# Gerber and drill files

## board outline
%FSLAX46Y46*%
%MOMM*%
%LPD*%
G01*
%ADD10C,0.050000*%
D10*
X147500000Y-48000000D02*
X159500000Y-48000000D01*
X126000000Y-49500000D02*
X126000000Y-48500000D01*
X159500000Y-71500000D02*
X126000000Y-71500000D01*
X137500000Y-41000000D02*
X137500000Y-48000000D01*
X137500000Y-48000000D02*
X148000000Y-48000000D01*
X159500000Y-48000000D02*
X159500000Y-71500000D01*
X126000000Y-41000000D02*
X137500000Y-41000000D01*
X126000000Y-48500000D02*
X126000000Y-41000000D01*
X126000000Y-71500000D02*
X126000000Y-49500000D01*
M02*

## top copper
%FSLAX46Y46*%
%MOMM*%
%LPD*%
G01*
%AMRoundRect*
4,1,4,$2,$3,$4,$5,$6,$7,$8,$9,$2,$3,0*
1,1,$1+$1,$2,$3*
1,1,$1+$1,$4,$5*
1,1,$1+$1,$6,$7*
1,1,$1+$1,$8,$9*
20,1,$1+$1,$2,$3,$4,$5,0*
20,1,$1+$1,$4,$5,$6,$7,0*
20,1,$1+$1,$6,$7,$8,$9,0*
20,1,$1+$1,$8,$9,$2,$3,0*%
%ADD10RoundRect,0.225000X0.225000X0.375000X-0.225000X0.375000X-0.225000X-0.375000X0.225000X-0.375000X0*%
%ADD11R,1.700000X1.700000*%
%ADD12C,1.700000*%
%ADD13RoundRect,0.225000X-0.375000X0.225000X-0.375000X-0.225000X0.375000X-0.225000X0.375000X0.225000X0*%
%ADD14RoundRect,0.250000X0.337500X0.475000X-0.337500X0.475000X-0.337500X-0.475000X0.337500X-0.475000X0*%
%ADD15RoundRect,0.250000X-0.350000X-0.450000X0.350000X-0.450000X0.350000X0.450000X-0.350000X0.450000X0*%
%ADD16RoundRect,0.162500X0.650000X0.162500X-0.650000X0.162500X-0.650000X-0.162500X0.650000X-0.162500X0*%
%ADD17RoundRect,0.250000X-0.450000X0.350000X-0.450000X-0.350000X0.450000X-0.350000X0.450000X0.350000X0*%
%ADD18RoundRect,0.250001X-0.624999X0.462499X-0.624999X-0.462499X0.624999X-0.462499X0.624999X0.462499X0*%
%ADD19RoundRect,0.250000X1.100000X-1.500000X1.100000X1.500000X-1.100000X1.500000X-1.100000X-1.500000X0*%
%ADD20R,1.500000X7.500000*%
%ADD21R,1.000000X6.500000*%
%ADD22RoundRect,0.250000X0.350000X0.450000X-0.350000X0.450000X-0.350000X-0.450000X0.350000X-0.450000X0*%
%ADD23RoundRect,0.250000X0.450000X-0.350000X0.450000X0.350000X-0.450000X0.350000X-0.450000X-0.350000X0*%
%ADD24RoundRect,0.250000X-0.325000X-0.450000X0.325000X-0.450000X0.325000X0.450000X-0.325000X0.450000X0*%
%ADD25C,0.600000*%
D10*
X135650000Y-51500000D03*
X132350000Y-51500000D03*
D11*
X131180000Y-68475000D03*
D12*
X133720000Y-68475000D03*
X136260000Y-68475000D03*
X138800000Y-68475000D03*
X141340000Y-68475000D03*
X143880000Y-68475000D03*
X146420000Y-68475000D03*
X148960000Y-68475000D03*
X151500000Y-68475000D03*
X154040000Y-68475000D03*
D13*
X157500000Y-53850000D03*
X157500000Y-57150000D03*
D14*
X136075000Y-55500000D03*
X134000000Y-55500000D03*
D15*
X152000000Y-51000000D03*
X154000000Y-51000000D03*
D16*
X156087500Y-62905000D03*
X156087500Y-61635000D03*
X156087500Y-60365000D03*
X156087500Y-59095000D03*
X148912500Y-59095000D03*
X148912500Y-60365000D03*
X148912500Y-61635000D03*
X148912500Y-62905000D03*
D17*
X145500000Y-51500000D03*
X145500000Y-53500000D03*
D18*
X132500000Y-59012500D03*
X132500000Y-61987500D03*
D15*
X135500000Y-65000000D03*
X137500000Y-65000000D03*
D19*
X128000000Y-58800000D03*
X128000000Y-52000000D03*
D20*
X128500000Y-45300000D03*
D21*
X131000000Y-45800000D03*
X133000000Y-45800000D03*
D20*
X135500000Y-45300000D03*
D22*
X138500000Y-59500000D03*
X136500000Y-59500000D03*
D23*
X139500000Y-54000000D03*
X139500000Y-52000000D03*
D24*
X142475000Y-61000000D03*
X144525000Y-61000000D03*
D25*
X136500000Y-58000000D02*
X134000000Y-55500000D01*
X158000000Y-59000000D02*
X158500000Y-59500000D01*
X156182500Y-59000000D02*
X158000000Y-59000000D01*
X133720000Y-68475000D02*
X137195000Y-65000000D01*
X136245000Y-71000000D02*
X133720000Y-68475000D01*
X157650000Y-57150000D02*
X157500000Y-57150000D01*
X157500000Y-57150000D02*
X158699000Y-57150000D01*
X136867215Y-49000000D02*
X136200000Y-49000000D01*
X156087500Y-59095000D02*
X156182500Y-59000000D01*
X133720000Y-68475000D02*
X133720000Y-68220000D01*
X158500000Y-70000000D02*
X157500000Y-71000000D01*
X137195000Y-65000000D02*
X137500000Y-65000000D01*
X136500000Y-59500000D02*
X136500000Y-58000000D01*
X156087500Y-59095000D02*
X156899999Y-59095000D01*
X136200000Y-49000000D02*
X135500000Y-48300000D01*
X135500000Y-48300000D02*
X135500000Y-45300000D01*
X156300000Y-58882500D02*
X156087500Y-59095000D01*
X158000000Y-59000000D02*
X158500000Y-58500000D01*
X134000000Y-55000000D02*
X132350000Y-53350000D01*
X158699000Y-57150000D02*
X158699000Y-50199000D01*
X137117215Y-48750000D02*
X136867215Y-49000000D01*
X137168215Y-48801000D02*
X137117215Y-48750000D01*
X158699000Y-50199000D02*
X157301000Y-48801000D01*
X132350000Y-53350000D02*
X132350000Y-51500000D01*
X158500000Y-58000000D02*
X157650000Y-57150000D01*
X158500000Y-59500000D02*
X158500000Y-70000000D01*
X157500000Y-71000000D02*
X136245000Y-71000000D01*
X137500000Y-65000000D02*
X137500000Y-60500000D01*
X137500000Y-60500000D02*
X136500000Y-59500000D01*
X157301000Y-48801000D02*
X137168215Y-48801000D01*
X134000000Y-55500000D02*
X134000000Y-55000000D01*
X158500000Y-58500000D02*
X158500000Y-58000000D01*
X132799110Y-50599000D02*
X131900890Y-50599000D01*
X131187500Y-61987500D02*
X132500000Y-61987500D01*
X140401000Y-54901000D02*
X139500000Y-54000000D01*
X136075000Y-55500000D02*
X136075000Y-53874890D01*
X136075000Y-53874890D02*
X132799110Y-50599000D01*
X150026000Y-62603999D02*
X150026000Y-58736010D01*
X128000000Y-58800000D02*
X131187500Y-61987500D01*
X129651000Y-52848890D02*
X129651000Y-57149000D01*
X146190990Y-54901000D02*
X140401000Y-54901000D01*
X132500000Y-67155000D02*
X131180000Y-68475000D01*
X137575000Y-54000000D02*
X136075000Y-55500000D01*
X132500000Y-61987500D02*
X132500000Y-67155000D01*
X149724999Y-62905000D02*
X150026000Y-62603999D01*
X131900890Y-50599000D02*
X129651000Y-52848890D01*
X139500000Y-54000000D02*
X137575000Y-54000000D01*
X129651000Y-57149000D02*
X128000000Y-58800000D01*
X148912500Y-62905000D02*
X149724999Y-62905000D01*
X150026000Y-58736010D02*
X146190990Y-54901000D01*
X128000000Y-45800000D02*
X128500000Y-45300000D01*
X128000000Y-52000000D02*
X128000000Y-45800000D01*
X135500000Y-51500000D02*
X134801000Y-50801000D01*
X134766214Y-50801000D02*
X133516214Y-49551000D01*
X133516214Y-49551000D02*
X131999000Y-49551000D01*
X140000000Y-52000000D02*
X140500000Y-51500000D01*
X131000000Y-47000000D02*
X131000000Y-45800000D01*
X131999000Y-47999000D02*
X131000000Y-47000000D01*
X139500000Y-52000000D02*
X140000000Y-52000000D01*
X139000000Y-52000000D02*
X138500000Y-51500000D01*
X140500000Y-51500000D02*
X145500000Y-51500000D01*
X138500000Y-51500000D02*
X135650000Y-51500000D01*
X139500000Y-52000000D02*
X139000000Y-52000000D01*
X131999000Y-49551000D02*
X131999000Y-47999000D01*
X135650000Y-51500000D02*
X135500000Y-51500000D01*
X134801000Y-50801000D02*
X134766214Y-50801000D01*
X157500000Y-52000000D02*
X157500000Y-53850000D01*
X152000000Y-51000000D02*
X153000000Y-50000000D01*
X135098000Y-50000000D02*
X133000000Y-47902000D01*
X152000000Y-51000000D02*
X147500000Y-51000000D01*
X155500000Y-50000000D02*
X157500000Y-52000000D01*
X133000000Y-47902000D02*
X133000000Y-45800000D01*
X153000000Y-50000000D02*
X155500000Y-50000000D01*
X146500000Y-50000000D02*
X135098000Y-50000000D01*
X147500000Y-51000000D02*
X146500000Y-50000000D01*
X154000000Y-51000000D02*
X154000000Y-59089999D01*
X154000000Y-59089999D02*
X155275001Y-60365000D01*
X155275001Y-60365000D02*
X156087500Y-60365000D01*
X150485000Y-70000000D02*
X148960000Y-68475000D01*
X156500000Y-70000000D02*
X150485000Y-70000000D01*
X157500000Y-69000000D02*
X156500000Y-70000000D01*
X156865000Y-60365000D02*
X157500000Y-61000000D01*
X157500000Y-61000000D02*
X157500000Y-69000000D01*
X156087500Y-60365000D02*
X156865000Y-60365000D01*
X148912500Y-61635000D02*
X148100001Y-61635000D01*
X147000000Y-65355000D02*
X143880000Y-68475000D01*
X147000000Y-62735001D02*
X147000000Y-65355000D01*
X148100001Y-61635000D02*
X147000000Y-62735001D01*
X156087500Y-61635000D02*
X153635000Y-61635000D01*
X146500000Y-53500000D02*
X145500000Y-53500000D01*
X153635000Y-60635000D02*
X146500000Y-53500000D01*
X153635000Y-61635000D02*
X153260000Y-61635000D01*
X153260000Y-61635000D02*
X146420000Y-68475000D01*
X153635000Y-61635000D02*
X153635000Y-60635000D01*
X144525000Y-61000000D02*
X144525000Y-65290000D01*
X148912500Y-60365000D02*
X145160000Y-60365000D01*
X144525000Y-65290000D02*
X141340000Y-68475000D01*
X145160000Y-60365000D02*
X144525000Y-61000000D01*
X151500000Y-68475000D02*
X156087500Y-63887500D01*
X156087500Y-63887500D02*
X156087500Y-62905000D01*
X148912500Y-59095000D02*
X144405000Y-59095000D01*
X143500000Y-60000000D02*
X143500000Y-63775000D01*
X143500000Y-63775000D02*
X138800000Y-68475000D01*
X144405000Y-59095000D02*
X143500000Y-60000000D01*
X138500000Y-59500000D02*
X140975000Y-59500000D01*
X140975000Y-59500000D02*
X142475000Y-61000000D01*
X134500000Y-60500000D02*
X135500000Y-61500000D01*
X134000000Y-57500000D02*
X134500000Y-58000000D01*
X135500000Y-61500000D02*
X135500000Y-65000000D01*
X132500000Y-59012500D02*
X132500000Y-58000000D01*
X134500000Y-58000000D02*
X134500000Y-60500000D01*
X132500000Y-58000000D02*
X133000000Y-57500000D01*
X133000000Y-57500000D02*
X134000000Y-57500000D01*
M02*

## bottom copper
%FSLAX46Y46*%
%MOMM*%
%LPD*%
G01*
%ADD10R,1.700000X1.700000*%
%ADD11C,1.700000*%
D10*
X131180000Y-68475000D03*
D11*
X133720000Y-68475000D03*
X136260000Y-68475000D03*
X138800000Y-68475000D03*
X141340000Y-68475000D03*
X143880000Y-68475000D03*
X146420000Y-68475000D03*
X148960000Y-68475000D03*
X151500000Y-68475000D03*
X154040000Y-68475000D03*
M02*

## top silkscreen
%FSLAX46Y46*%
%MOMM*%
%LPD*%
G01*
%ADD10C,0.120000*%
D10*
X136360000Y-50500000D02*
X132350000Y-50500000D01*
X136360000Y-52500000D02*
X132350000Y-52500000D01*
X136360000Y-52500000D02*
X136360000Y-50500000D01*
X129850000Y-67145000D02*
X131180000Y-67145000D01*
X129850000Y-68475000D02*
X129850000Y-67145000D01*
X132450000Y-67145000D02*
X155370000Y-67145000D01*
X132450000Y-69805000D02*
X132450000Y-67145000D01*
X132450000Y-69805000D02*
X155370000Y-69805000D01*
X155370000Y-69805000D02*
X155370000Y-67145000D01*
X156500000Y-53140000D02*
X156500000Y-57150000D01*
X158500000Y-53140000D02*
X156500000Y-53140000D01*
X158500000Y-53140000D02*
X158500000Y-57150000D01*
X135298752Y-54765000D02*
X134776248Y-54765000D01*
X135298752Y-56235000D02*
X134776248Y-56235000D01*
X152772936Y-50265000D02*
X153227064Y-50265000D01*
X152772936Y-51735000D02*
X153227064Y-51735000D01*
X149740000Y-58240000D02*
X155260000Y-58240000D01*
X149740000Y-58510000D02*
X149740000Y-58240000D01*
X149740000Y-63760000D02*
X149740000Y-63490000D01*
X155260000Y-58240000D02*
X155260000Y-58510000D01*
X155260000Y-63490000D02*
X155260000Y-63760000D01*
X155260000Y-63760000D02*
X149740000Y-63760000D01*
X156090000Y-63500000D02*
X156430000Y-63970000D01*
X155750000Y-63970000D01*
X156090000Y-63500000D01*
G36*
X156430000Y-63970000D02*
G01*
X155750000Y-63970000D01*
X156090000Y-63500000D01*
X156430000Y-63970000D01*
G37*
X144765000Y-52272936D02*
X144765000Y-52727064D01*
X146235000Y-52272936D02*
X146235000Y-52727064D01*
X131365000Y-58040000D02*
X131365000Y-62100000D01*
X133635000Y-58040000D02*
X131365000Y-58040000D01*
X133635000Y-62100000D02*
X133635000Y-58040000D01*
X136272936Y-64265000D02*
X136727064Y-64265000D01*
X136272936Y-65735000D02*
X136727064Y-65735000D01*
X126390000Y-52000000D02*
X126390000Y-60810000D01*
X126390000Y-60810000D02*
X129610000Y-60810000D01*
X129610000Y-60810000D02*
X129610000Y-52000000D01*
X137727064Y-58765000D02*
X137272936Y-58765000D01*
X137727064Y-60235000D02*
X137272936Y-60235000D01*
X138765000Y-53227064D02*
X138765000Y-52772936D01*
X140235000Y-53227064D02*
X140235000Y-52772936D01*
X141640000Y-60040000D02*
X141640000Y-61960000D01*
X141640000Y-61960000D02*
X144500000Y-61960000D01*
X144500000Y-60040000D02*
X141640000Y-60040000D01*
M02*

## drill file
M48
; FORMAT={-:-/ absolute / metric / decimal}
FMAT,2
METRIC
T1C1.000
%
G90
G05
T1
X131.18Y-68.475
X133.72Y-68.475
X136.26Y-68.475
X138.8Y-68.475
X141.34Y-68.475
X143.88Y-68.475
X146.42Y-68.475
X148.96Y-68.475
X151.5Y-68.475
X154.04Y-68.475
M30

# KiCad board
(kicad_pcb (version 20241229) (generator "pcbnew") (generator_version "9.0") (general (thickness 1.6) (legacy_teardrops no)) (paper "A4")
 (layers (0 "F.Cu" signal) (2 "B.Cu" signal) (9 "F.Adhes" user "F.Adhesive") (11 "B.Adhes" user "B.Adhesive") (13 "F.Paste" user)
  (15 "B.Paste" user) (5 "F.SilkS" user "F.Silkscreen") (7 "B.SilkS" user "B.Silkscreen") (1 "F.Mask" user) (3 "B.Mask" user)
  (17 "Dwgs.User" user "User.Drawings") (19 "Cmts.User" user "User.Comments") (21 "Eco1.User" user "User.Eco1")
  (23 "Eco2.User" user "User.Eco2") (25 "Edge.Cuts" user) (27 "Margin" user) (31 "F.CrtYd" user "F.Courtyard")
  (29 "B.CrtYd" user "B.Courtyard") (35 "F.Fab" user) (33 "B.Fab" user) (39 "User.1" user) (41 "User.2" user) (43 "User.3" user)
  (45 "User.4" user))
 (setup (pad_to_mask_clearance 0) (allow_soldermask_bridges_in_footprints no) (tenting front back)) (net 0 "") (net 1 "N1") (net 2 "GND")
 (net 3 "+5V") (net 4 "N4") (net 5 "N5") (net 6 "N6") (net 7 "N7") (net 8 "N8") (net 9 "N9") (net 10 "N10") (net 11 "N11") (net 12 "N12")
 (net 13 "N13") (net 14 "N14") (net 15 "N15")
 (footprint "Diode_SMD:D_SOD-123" (layer "F.Cu") (at 134 51.5 180)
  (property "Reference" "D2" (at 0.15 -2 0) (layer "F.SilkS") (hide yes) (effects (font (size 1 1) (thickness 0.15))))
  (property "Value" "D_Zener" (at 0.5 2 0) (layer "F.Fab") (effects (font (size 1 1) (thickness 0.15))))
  (fp_line (start -2.36 1) (end 1.65 1) (stroke (width 0.12) (type solid)) (layer "F.SilkS"))
  (fp_line (start -2.36 -1) (end 1.65 -1) (stroke (width 0.12) (type solid)) (layer "F.SilkS"))
  (fp_line (start -2.36 -1) (end -2.36 1) (stroke (width 0.12) (type solid)) (layer "F.SilkS"))
  (pad "1" smd roundrect (at -1.65 0 180) (size 0.9 1.2) (layers "F.Cu" "F.Mask" "F.Paste") (roundrect_rratio 0.25) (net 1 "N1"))
  (pad "2" smd roundrect (at 1.65 0 180) (size 0.9 1.2) (layers "F.Cu" "F.Mask" "F.Paste") (roundrect_rratio 0.25) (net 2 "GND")))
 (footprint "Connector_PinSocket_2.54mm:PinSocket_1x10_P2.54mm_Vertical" (layer "F.Cu") (at 131.18 68.475 90)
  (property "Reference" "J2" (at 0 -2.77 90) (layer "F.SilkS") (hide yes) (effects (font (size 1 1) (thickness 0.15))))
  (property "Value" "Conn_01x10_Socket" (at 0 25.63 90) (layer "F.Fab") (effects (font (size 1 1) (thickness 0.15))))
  (fp_line (start 1.33 -1.33) (end 1.33 0) (stroke (width 0.12) (type solid)) (layer "F.SilkS"))
  (fp_line (start 0 -1.33) (end 1.33 -1.33) (stroke (width 0.12) (type solid)) (layer "F.SilkS"))
  (fp_line (start 1.33 1.27) (end 1.33 24.19) (stroke (width 0.12) (type solid)) (layer "F.SilkS"))
  (fp_line (start -1.33 1.27) (end 1.33 1.27) (stroke (width 0.12) (type solid)) (layer "F.SilkS"))
  (fp_line (start -1.33 1.27) (end -1.33 24.19) (stroke (width 0.12) (type solid)) (layer "F.SilkS"))
  (fp_line (start -1.33 24.19) (end 1.33 24.19) (stroke (width 0.12) (type solid)) (layer "F.SilkS"))
  (pad "1" thru_hole rect (at 0 0 90) (size 1.7 1.7) (drill 1) (layers "*.Cu" "*.Mask") (remove_unused_layers no) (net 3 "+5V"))
  (pad "2" thru_hole circle (at 0 2.54 90) (size 1.7 1.7) (drill 1) (layers "*.Cu" "*.Mask") (remove_unused_layers no) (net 2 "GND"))
  (pad "3" thru_hole circle (at 0 5.08 90) (size 1.7 1.7) (drill 1) (layers "*.Cu" "*.Mask") (remove_unused_layers no) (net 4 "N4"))
  (pad "4" thru_hole circle (at 0 7.62 90) (size 1.7 1.7) (drill 1) (layers "*.Cu" "*.Mask") (remove_unused_layers no) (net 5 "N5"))
  (pad "5" thru_hole circle (at 0 10.16 90) (size 1.7 1.7) (drill 1) (layers "*.Cu" "*.Mask") (remove_unused_layers no) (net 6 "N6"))
  (pad "6" thru_hole circle (at 0 12.7 90) (size 1.7 1.7) (drill 1) (layers "*.Cu" "*.Mask") (remove_unused_layers no) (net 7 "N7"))
  (pad "7" thru_hole circle (at 0 15.24 90) (size 1.7 1.7) (drill 1) (layers "*.Cu" "*.Mask") (remove_unused_layers no) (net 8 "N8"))
  (pad "8" thru_hole circle (at 0 17.78 90) (size 1.7 1.7) (drill 1) (layers "*.Cu" "*.Mask") (remove_unused_layers no) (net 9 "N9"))
  (pad "9" thru_hole circle (at 0 20.32 90) (size 1.7 1.7) (drill 1) (layers "*.Cu" "*.Mask") (remove_unused_layers no) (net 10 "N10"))
  (pad "10" thru_hole circle (at 0 22.86 90) (size 1.7 1.7) (drill 1) (layers "*.Cu" "*.Mask") (remove_unused_layers no) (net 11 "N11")))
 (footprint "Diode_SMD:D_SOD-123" (layer "F.Cu") (at 157.5 55.5 -90)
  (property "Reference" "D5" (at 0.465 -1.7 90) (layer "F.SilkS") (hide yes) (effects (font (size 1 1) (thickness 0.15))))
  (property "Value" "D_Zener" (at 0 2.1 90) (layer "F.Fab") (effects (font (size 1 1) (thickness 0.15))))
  (fp_line (start -2.36 1) (end 1.65 1) (stroke (width 0.12) (type solid)) (layer "F.SilkS"))
  (fp_line (start -2.36 -1) (end -2.36 1) (stroke (width 0.12) (type solid)) (layer "F.SilkS"))
  (fp_line (start -2.36 -1) (end 1.65 -1) (stroke (width 0.12) (type solid)) (layer "F.SilkS"))
  (pad "1" smd roundrect (at -1.65 0 270) (size 0.9 1.2) (layers "F.Cu" "F.Mask" "F.Paste") (roundrect_rratio 0.25) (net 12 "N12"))
  (pad "2" smd roundrect (at 1.65 0 270) (size 0.9 1.2) (layers "F.Cu" "F.Mask" "F.Paste") (roundrect_rratio 0.25) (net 2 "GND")))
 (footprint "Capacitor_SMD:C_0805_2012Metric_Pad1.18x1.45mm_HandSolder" (layer "F.Cu") (at 135.0375 55.5 180)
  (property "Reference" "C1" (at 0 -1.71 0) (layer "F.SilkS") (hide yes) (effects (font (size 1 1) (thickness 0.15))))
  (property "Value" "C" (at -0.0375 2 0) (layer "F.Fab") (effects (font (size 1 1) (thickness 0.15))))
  (fp_line (start -0.261252 0.735) (end 0.261252 0.735) (stroke (width 0.12) (type solid)) (layer "F.SilkS"))
  (fp_line (start -0.261252 -0.735) (end 0.261252 -0.735) (stroke (width 0.12) (type solid)) (layer "F.SilkS"))
  (pad "1" smd roundrect (at -1.0375 0 180) (size 1.175 1.45) (layers "F.Cu" "F.Mask" "F.Paste") (roundrect_rratio 0.212766) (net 3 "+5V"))
  (pad "2" smd roundrect (at 1.0375 0 180) (size 1.175 1.45) (layers "F.Cu" "F.Mask" "F.Paste") (roundrect_rratio 0.212766) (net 2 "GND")))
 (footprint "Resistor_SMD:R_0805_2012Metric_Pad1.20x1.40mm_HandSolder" (layer "F.Cu") (at 153 51)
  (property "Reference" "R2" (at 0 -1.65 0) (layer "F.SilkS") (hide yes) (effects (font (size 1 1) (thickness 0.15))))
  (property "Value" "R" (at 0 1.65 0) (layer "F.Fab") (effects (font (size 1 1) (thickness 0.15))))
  (fp_line (start -0.227064 -0.735) (end 0.227064 -0.735) (stroke (width 0.12) (type solid)) (layer "F.SilkS"))
  (fp_line (start -0.227064 0.735) (end 0.227064 0.735) (stroke (width 0.12) (type solid)) (layer "F.SilkS"))
  (pad "1" smd roundrect (at -1 0) (size 1.2 1.4) (layers "F.Cu" "F.Mask" "F.Paste") (roundrect_rratio 0.208333) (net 12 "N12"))
  (pad "2" smd roundrect (at 1 0) (size 1.2 1.4) (layers "F.Cu" "F.Mask" "F.Paste") (roundrect_rratio 0.208333) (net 9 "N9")))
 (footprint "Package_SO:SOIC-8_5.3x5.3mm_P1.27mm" (layer "F.Cu") (at 152.5 61 180)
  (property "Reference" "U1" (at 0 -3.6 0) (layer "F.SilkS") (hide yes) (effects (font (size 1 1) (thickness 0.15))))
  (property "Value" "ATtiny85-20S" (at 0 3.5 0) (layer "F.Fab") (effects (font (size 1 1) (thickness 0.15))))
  (fp_line (start 2.76 2.76) (end -2.76 2.76) (stroke (width 0.12) (type solid)) (layer "F.SilkS"))
  (fp_line (start 2.76 2.49) (end 2.76 2.76) (stroke (width 0.12) (type solid)) (layer "F.SilkS"))
  (fp_line (start 2.76 -2.76) (end 2.76 -2.49) (stroke (width 0.12) (type solid)) (layer "F.SilkS"))
  (fp_line (start -2.76 2.76) (end -2.76 2.49) (stroke (width 0.12) (type solid)) (layer "F.SilkS"))
  (fp_line (start -2.76 -2.49) (end -2.76 -2.76) (stroke (width 0.12) (type solid)) (layer "F.SilkS"))
  (fp_line (start -2.76 -2.76) (end 2.76 -2.76) (stroke (width 0.12) (type solid)) (layer "F.SilkS"))
  (fp_poly (pts (xy -3.59 -2.5) (xy -3.93 -2.97) (xy -3.25 -2.97)) (stroke (width 0.12) (type solid)) (fill yes) (layer "F.SilkS"))
  (pad "1" smd roundrect (at -3.5875 -1.905 180) (size 1.625 0.65) (layers "F.Cu" "F.Mask" "F.Paste") (roundrect_rratio 0.25) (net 10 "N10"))
  (pad "2" smd roundrect (at -3.5875 -0.635 180) (size 1.625 0.65) (layers "F.Cu" "F.Mask" "F.Paste") (roundrect_rratio 0.25) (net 8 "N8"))
  (pad "3" smd roundrect (at -3.5875 0.635 180) (size 1.625 0.65) (layers "F.Cu" "F.Mask" "F.Paste") (roundrect_rratio 0.25) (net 9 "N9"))
  (pad "4" smd roundrect (at -3.5875 1.905 180) (size 1.625 0.65) (layers "F.Cu" "F.Mask" "F.Paste") (roundrect_rratio 0.25) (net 2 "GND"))
  (pad "5" smd roundrect (at 3.5875 1.905 180) (size 1.625 0.65) (layers "F.Cu" "F.Mask" "F.Paste") (roundrect_rratio 0.25) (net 5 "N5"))
  (pad "6" smd roundrect (at 3.5875 0.635 180) (size 1.625 0.65) (layers "F.Cu" "F.Mask" "F.Paste") (roundrect_rratio 0.25) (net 6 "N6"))
  (pad "7" smd roundrect (at 3.5875 -0.635 180) (size 1.625 0.65) (layers "F.Cu" "F.Mask" "F.Paste") (roundrect_rratio 0.25) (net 7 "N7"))
  (pad "8" smd roundrect (at 3.5875 -1.905 180) (size 1.625 0.65) (layers "F.Cu" "F.Mask" "F.Paste") (roundrect_rratio 0.25) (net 3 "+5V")))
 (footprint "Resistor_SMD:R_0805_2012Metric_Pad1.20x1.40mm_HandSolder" (layer "F.Cu") (at 145.5 52.5 -90)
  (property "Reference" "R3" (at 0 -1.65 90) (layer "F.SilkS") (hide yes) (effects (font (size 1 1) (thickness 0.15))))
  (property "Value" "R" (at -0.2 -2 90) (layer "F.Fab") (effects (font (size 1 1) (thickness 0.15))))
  (fp_line (start -0.227064 0.735) (end 0.227064 0.735) (stroke (width 0.12) (type solid)) (layer "F.SilkS"))
  (fp_line (start -0.227064 -0.735) (end 0.227064 -0.735) (stroke (width 0.12) (type solid)) (layer "F.SilkS"))
  (pad "1" smd roundrect (at -1 0 270) (size 1.2 1.4) (layers "F.Cu" "F.Mask" "F.Paste") (roundrect_rratio 0.208333) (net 1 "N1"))
  (pad "2" smd roundrect (at 1 0 270) (size 1.2 1.4) (layers "F.Cu" "F.Mask" "F.Paste") (roundrect_rratio 0.208333) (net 8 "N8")))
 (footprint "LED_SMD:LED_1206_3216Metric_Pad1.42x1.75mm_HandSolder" (layer "F.Cu") (at 132.5 60.5 -90)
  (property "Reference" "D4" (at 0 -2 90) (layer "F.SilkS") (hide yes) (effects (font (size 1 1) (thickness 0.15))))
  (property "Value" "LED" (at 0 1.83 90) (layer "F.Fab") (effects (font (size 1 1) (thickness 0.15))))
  (fp_line (start -2.46 1.135) (end 1.6 1.135) (stroke (width 0.12) (type solid)) (layer "F.SilkS"))
  (fp_line (start -2.46 -1.135) (end -2.46 1.135) (stroke (width 0.12) (type solid)) (layer "F.SilkS"))
  (fp_line (start 1.6 -1.135) (end -2.46 -1.135) (stroke (width 0.12) (type solid)) (layer "F.SilkS"))
  (pad "1" smd roundrect (at -1.4875 0 270) (size 1.425 1.75) (layers "F.Cu" "F.Mask" "F.Paste") (roundrect_rratio 0.175439) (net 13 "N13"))
  (pad "2" smd roundrect (at 1.4875 0 270) (size 1.425 1.75) (layers "F.Cu" "F.Mask" "F.Paste") (roundrect_rratio 0.175439) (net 3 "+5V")))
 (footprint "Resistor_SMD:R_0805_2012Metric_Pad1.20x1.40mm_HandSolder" (layer "F.Cu") (at 136.5 65)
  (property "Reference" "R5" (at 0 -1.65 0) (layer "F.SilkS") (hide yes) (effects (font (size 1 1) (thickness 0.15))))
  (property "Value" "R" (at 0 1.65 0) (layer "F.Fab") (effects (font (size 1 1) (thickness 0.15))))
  (fp_line (start -0.227064 -0.735) (end 0.227064 -0.735) (stroke (width 0.12) (type solid)) (layer "F.SilkS"))
  (fp_line (start -0.227064 0.735) (end 0.227064 0.735) (stroke (width 0.12) (type solid)) (layer "F.SilkS"))
  (pad "1" smd roundrect (at -1 0) (size 1.2 1.4) (layers "F.Cu" "F.Mask" "F.Paste") (roundrect_rratio 0.208333) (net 13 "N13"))
  (pad "2" smd roundrect (at 1 0) (size 1.2 1.4) (layers "F.Cu" "F.Mask" "F.Paste") (roundrect_rratio 0.208333) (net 2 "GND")))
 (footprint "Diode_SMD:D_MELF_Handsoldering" (layer "F.Cu") (at 128 55.4 90)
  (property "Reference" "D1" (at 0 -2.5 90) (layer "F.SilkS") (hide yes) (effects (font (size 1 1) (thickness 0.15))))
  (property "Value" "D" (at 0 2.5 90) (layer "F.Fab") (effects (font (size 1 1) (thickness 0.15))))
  (fp_line (start 3.4 -1.61) (end -5.41 -1.61) (stroke (width 0.12) (type solid)) (layer "F.SilkS"))
  (fp_line (start -5.41 -1.61) (end -5.41 1.61) (stroke (width 0.12) (type solid)) (layer "F.SilkS"))
  (fp_line (start -5.41 1.61) (end 3.4 1.61) (stroke (width 0.12) (type solid)) (layer "F.SilkS"))
  (pad "1" smd roundrect (at -3.4 0 90) (size 3.5 2.7) (layers "F.Cu" "F.Mask" "F.Paste") (roundrect_rratio 0.0925925926) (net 3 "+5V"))
  (pad "2" smd roundrect (at 3.4 0 90) (size 3.5 2.7) (layers "F.Cu" "F.Mask" "F.Paste") (roundrect_rratio 0.0925925926) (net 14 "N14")))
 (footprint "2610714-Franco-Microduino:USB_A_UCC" (layer "F.Cu") (at 132 45.5 -90)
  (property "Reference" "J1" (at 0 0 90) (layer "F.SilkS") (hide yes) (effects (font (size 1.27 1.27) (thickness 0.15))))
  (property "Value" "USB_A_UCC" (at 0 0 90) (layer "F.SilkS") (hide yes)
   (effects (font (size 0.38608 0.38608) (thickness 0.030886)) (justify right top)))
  (pad "1" smd rect (at -0.2 3.5 270) (size 7.5 1.5) (layers "F.Cu" "F.Mask" "F.Paste") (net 14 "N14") (solder_mask_margin 0.1016))
  (pad "2" smd rect (at 0.3 1 270) (size 6.5 1) (layers "F.Cu" "F.Mask" "F.Paste") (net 1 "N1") (solder_mask_margin 0.1016))
  (pad "3" smd rect (at 0.3 -1 270) (size 6.5 1) (layers "F.Cu" "F.Mask" "F.Paste") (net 12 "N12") (solder_mask_margin 0.1016))
  (pad "4" smd rect (at -0.2 -3.5 270) (size 7.5 1.5) (layers "F.Cu" "F.Mask" "F.Paste") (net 2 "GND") (solder_mask_margin 0.1016)))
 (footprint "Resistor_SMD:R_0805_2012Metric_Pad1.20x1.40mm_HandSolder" (layer "F.Cu") (at 137.5 59.5 180)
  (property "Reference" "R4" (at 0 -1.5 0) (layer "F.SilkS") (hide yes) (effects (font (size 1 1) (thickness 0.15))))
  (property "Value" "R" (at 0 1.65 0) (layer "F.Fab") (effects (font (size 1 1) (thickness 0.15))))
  (fp_line (start -0.227064 0.735) (end 0.227064 0.735) (stroke (width 0.12) (type solid)) (layer "F.SilkS"))
  (fp_line (start -0.227064 -0.735) (end 0.227064 -0.735) (stroke (width 0.12) (type solid)) (layer "F.SilkS"))
  (pad "1" smd roundrect (at -1 0 180) (size 1.2 1.4) (layers "F.Cu" "F.Mask" "F.Paste") (roundrect_rratio 0.208333) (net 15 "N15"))
  (pad "2" smd roundrect (at 1 0 180) (size 1.2 1.4) (layers "F.Cu" "F.Mask" "F.Paste") (roundrect_rratio 0.208333) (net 2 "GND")))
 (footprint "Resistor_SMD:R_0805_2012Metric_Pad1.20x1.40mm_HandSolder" (layer "F.Cu") (at 139.5 53 90)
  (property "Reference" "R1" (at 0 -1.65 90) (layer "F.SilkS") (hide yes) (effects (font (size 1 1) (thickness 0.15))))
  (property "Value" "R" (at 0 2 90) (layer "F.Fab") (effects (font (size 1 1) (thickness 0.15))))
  (fp_line (start -0.227064 -0.735) (end 0.227064 -0.735) (stroke (width 0.12) (type solid)) (layer "F.SilkS"))
  (fp_line (start -0.227064 0.735) (end 0.227064 0.735) (stroke (width 0.12) (type solid)) (layer "F.SilkS"))
  (pad "1" smd roundrect (at -1 0 90) (size 1.2 1.4) (layers "F.Cu" "F.Mask" "F.Paste") (roundrect_rratio 0.208333) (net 3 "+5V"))
  (pad "2" smd roundrect (at 1 0 90) (size 1.2 1.4) (layers "F.Cu" "F.Mask" "F.Paste") (roundrect_rratio 0.208333) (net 1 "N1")))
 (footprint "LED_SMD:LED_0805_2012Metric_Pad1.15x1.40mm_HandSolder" (layer "F.Cu") (at 143.5 61)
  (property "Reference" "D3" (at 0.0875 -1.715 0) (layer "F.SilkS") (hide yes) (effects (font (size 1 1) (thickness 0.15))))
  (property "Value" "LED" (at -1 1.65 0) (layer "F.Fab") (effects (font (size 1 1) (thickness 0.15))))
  (fp_line (start -1.86 -0.96) (end -1.86 0.96) (stroke (width 0.12) (type solid)) (layer "F.SilkS"))
  (fp_line (start -1.86 0.96) (end 1 0.96) (stroke (width 0.12) (type solid)) (layer "F.SilkS"))
  (fp_line (start 1 -0.96) (end -1.86 -0.96) (stroke (width 0.12) (type solid)) (layer "F.SilkS"))
  (pad "1" smd roundrect (at -1.025 0) (size 1.15 1.4) (layers "F.Cu" "F.Mask" "F.Paste") (roundrect_rratio 0.217391) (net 15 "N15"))
  (pad "2" smd roundrect (at 1.025 0) (size 1.15 1.4) (layers "F.Cu" "F.Mask" "F.Paste") (roundrect_rratio 0.217391) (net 6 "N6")))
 (gr_line (start 147.5 48) (end 159.5 48) (stroke (width 0.05) (type default)) (layer "Edge.Cuts"))
 (gr_line (start 126 49.5) (end 126 48.5) (stroke (width 0.05) (type default)) (layer "Edge.Cuts"))
 (gr_line (start 159.5 71.5) (end 126 71.5) (stroke (width 0.05) (type default)) (layer "Edge.Cuts"))
 (gr_line (start 137.5 41) (end 137.5 48) (stroke (width 0.05) (type default)) (layer "Edge.Cuts"))
 (gr_line (start 137.5 48) (end 148 48) (stroke (width 0.05) (type default)) (layer "Edge.Cuts"))
 (gr_line (start 159.5 48) (end 159.5 71.5) (stroke (width 0.05) (type default)) (layer "Edge.Cuts"))
 (gr_line (start 126 41) (end 137.5 41) (stroke (width 0.05) (type default)) (layer "Edge.Cuts"))
 (gr_line (start 126 48.5) (end 126 41) (stroke (width 0.05) (type default)) (layer "Edge.Cuts"))
 (gr_line (start 126 71.5) (end 126 49.5) (stroke (width 0.05) (type default)) (layer "Edge.Cuts"))
 (segment (start 136.5 58) (end 134 55.5) (width 0.6) (layer "F.Cu") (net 2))
 (segment (start 158 59) (end 158.5 59.5) (width 0.6) (layer "F.Cu") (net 2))
 (segment (start 156.1825 59) (end 158 59) (width 0.6) (layer "F.Cu") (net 2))
 (segment (start 133.72 68.475) (end 137.195 65) (width 0.6) (layer "F.Cu") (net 2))
 (segment (start 136.245 71) (end 133.72 68.475) (width 0.6) (layer "F.Cu") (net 2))
 (segment (start 157.65 57.15) (end 157.5 57.15) (width 0.6) (layer "F.Cu") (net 2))
 (segment (start 157.5 57.15) (end 158.699 57.15) (width 0.6) (layer "F.Cu") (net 2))
 (segment (start 136.867215 49) (end 136.2 49) (width 0.6) (layer "F.Cu") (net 2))
 (segment (start 156.0875 59.095) (end 156.1825 59) (width 0.6) (layer "F.Cu") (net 2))
 (segment (start 133.72 68.475) (end 133.72 68.22) (width 0.6) (layer "F.Cu") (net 2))
 (segment (start 158.5 70) (end 157.5 71) (width 0.6) (layer "F.Cu") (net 2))
 (segment (start 137.195 65) (end 137.5 65) (width 0.6) (layer "F.Cu") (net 2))
 (segment (start 136.5 59.5) (end 136.5 58) (width 0.6) (layer "F.Cu") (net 2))
 (segment (start 156.0875 59.095) (end 156.899999 59.095) (width 0.6) (layer "F.Cu") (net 2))
 (segment (start 136.2 49) (end 135.5 48.3) (width 0.6) (layer "F.Cu") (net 2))
 (segment (start 135.5 48.3) (end 135.5 45.3) (width 0.6) (layer "F.Cu") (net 2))
 (segment (start 156.3 58.8825) (end 156.0875 59.095) (width 0.6) (layer "F.Cu") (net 2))
 (segment (start 158 59) (end 158.5 58.5) (width 0.6) (layer "F.Cu") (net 2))
 (segment (start 134 55) (end 132.35 53.35) (width 0.6) (layer "F.Cu") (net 2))
 (segment (start 158.699 57.15) (end 158.699 50.199) (width 0.6) (layer "F.Cu") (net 2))
 (segment (start 137.117215 48.75) (end 136.867215 49) (width 0.6) (layer "F.Cu") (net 2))
 (segment (start 137.168215 48.801) (end 137.117215 48.75) (width 0.6) (layer "F.Cu") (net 2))
 (segment (start 158.699 50.199) (end 157.301 48.801) (width 0.6) (layer "F.Cu") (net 2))
 (segment (start 132.35 53.35) (end 132.35 51.5) (width 0.6) (layer "F.Cu") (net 2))
 (segment (start 158.5 58) (end 157.65 57.15) (width 0.6) (layer "F.Cu") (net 2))
 (segment (start 158.5 59.5) (end 158.5 70) (width 0.6) (layer "F.Cu") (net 2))
 (segment (start 157.5 71) (end 136.245 71) (width 0.6) (layer "F.Cu") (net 2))
 (segment (start 137.5 65) (end 137.5 60.5) (width 0.6) (layer "F.Cu") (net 2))
 (segment (start 137.5 60.5) (end 136.5 59.5) (width 0.6) (layer "F.Cu") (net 2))
 (segment (start 157.301 48.801) (end 137.168215 48.801) (width 0.6) (layer "F.Cu") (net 2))
 (segment (start 134 55.5) (end 134 55) (width 0.6) (layer "F.Cu") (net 2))
 (segment (start 158.5 58.5) (end 158.5 58) (width 0.6) (layer "F.Cu") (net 2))
 (segment (start 132.79911 50.599) (end 131.90089 50.599) (width 0.6) (layer "F.Cu") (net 3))
 (segment (start 131.1875 61.9875) (end 132.5 61.9875) (width 0.6) (layer "F.Cu") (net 3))
 (segment (start 140.401 54.901) (end 139.5 54) (width 0.6) (layer "F.Cu") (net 3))
 (segment (start 136.075 55.5) (end 136.075 53.87489) (width 0.6) (layer "F.Cu") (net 3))
 (segment (start 136.075 53.87489) (end 132.79911 50.599) (width 0.6) (layer "F.Cu") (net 3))
 (segment (start 150.026 62.603999) (end 150.026 58.73601) (width 0.6) (layer "F.Cu") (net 3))
 (segment (start 128 58.8) (end 131.1875 61.9875) (width 0.6) (layer "F.Cu") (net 3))
 (segment (start 129.651 52.84889) (end 129.651 57.149) (width 0.6) (layer "F.Cu") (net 3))
 (segment (start 146.19099 54.901) (end 140.401 54.901) (width 0.6) (layer "F.Cu") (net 3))
 (segment (start 132.5 67.155) (end 131.18 68.475) (width 0.6) (layer "F.Cu") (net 3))
 (segment (start 137.575 54) (end 136.075 55.5) (width 0.6) (layer "F.Cu") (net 3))
 (segment (start 132.5 61.9875) (end 132.5 67.155) (width 0.6) (layer "F.Cu") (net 3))
 (segment (start 149.724999 62.905) (end 150.026 62.603999) (width 0.6) (layer "F.Cu") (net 3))
 (segment (start 131.90089 50.599) (end 129.651 52.84889) (width 0.6) (layer "F.Cu") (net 3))
 (segment (start 139.5 54) (end 137.575 54) (width 0.6) (layer "F.Cu") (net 3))
 (segment (start 129.651 57.149) (end 128 58.8) (width 0.6) (layer "F.Cu") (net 3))
 (segment (start 148.9125 62.905) (end 149.724999 62.905) (width 0.6) (layer "F.Cu") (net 3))
 (segment (start 150.026 58.73601) (end 146.19099 54.901) (width 0.6) (layer "F.Cu") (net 3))
 (segment (start 128 45.8) (end 128.5 45.3) (width 0.6) (layer "F.Cu") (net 14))
 (segment (start 128 52) (end 128 45.8) (width 0.6) (layer "F.Cu") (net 14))
 (segment (start 135.5 51.5) (end 134.801 50.801) (width 0.6) (layer "F.Cu") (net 1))
 (segment (start 134.766214 50.801) (end 133.516214 49.551) (width 0.6) (layer "F.Cu") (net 1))
 (segment (start 133.516214 49.551) (end 131.999 49.551) (width 0.6) (layer "F.Cu") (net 1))
 (segment (start 140 52) (end 140.5 51.5) (width 0.6) (layer "F.Cu") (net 1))
 (segment (start 131 47) (end 131 45.8) (width 0.6) (layer "F.Cu") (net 1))
 (segment (start 131.999 47.999) (end 131 47) (width 0.6) (layer "F.Cu") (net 1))
 (segment (start 139.5 52) (end 140 52) (width 0.6) (layer "F.Cu") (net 1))
 (segment (start 139 52) (end 138.5 51.5) (width 0.6) (layer "F.Cu") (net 1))
 (segment (start 140.5 51.5) (end 145.5 51.5) (width 0.6) (layer "F.Cu") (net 1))
 (segment (start 138.5 51.5) (end 135.65 51.5) (width 0.6) (layer "F.Cu") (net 1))
 (segment (start 139.5 52) (end 139 52) (width 0.6) (layer "F.Cu") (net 1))
 (segment (start 131.999 49.551) (end 131.999 47.999) (width 0.6) (layer "F.Cu") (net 1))
 (segment (start 135.65 51.5) (end 135.5 51.5) (width 0.6) (layer "F.Cu") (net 1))
 (segment (start 134.801 50.801) (end 134.766214 50.801) (width 0.6) (layer "F.Cu") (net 1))
 (segment (start 157.5 52) (end 157.5 53.85) (width 0.6) (layer "F.Cu") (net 12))
 (segment (start 152 51) (end 153 50) (width 0.6) (layer "F.Cu") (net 12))
 (segment (start 135.098 50) (end 133 47.902) (width 0.6) (layer "F.Cu") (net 12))
 (segment (start 152 51) (end 147.5 51) (width 0.6) (layer "F.Cu") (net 12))
 (segment (start 155.5 50) (end 157.5 52) (width 0.6) (layer "F.Cu") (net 12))
 (segment (start 133 47.902) (end 133 45.8) (width 0.6) (layer "F.Cu") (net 12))
 (segment (start 153 50) (end 155.5 50) (width 0.6) (layer "F.Cu") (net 12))
 (segment (start 146.5 50) (end 135.098 50) (width 0.6) (layer "F.Cu") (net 12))
 (segment (start 147.5 51) (end 146.5 50) (width 0.6) (layer "F.Cu") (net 12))
 (segment (start 154 51) (end 154 59.089999) (width 0.6) (layer "F.Cu") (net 9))
 (segment (start 154 59.089999) (end 155.275001 60.365) (width 0.6) (layer "F.Cu") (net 9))
 (segment (start 155.275001 60.365) (end 156.0875 60.365) (width 0.6) (layer "F.Cu") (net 9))
 (segment (start 150.485 70) (end 148.96 68.475) (width 0.6) (layer "F.Cu") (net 9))
 (segment (start 156.5 70) (end 150.485 70) (width 0.6) (layer "F.Cu") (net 9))
 (segment (start 157.5 69) (end 156.5 70) (width 0.6) (layer "F.Cu") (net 9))
 (segment (start 156.865 60.365) (end 157.5 61) (width 0.6) (layer "F.Cu") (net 9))
 (segment (start 157.5 61) (end 157.5 69) (width 0.6) (layer "F.Cu") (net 9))
 (segment (start 156.0875 60.365) (end 156.865 60.365) (width 0.6) (layer "F.Cu") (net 9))
 (segment (start 148.9125 61.635) (end 148.100001 61.635) (width 0.6) (layer "F.Cu") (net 7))
 (segment (start 147 65.355) (end 143.88 68.475) (width 0.6) (layer "F.Cu") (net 7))
 (segment (start 147 62.735001) (end 147 65.355) (width 0.6) (layer "F.Cu") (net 7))
 (segment (start 148.100001 61.635) (end 147 62.735001) (width 0.6) (layer "F.Cu") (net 7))
 (segment (start 156.0875 61.635) (end 153.635 61.635) (width 0.6) (layer "F.Cu") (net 8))
 (segment (start 146.5 53.5) (end 145.5 53.5) (width 0.6) (layer "F.Cu") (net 8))
 (segment (start 153.635 60.635) (end 146.5 53.5) (width 0.6) (layer "F.Cu") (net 8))
 (segment (start 153.635 61.635) (end 153.26 61.635) (width 0.6) (layer "F.Cu") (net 8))
 (segment (start 153.26 61.635) (end 146.42 68.475) (width 0.6) (layer "F.Cu") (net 8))
 (segment (start 153.635 61.635) (end 153.635 60.635) (width 0.6) (layer "F.Cu") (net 8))
 (segment (start 144.525 61) (end 144.525 65.29) (width 0.6) (layer "F.Cu") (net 6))
 (segment (start 148.9125 60.365) (end 145.16 60.365) (width 0.6) (layer "F.Cu") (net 6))
 (segment (start 144.525 65.29) (end 141.34 68.475) (width 0.6) (layer "F.Cu") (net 6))
 (segment (start 145.16 60.365) (end 144.525 61) (width 0.6) (layer "F.Cu") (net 6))
 (segment (start 151.5 68.475) (end 156.0875 63.8875) (width 0.6) (layer "F.Cu") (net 10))
 (segment (start 156.0875 63.8875) (end 156.0875 62.905) (width 0.6) (layer "F.Cu") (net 10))
 (segment (start 148.9125 59.095) (end 144.405 59.095) (width 0.6) (layer "F.Cu") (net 5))
 (segment (start 143.5 60) (end 143.5 63.775) (width 0.6) (layer "F.Cu") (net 5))
 (segment (start 143.5 63.775) (end 138.8 68.475) (width 0.6) (layer "F.Cu") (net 5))
 (segment (start 144.405 59.095) (end 143.5 60) (width 0.6) (layer "F.Cu") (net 5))
 (segment (start 138.5 59.5) (end 140.975 59.5) (width 0.6) (layer "F.Cu") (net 15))
 (segment (start 140.975 59.5) (end 142.475 61) (width 0.6) (layer "F.Cu") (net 15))
 (segment (start 134.5 60.5) (end 135.5 61.5) (width 0.6) (layer "F.Cu") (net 13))
 (segment (start 134 57.5) (end 134.5 58) (width 0.6) (layer "F.Cu") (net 13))
 (segment (start 135.5 61.5) (end 135.5 65) (width 0.6) (layer "F.Cu") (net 13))
 (segment (start 132.5 59.0125) (end 132.5 58) (width 0.6) (layer "F.Cu") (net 13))
 (segment (start 134.5 58) (end 134.5 60.5) (width 0.6) (layer "F.Cu") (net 13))
 (segment (start 132.5 58) (end 133 57.5) (width 0.6) (layer "F.Cu") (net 13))
 (segment (start 133 57.5) (end 134 57.5) (width 0.6) (layer "F.Cu") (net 13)))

